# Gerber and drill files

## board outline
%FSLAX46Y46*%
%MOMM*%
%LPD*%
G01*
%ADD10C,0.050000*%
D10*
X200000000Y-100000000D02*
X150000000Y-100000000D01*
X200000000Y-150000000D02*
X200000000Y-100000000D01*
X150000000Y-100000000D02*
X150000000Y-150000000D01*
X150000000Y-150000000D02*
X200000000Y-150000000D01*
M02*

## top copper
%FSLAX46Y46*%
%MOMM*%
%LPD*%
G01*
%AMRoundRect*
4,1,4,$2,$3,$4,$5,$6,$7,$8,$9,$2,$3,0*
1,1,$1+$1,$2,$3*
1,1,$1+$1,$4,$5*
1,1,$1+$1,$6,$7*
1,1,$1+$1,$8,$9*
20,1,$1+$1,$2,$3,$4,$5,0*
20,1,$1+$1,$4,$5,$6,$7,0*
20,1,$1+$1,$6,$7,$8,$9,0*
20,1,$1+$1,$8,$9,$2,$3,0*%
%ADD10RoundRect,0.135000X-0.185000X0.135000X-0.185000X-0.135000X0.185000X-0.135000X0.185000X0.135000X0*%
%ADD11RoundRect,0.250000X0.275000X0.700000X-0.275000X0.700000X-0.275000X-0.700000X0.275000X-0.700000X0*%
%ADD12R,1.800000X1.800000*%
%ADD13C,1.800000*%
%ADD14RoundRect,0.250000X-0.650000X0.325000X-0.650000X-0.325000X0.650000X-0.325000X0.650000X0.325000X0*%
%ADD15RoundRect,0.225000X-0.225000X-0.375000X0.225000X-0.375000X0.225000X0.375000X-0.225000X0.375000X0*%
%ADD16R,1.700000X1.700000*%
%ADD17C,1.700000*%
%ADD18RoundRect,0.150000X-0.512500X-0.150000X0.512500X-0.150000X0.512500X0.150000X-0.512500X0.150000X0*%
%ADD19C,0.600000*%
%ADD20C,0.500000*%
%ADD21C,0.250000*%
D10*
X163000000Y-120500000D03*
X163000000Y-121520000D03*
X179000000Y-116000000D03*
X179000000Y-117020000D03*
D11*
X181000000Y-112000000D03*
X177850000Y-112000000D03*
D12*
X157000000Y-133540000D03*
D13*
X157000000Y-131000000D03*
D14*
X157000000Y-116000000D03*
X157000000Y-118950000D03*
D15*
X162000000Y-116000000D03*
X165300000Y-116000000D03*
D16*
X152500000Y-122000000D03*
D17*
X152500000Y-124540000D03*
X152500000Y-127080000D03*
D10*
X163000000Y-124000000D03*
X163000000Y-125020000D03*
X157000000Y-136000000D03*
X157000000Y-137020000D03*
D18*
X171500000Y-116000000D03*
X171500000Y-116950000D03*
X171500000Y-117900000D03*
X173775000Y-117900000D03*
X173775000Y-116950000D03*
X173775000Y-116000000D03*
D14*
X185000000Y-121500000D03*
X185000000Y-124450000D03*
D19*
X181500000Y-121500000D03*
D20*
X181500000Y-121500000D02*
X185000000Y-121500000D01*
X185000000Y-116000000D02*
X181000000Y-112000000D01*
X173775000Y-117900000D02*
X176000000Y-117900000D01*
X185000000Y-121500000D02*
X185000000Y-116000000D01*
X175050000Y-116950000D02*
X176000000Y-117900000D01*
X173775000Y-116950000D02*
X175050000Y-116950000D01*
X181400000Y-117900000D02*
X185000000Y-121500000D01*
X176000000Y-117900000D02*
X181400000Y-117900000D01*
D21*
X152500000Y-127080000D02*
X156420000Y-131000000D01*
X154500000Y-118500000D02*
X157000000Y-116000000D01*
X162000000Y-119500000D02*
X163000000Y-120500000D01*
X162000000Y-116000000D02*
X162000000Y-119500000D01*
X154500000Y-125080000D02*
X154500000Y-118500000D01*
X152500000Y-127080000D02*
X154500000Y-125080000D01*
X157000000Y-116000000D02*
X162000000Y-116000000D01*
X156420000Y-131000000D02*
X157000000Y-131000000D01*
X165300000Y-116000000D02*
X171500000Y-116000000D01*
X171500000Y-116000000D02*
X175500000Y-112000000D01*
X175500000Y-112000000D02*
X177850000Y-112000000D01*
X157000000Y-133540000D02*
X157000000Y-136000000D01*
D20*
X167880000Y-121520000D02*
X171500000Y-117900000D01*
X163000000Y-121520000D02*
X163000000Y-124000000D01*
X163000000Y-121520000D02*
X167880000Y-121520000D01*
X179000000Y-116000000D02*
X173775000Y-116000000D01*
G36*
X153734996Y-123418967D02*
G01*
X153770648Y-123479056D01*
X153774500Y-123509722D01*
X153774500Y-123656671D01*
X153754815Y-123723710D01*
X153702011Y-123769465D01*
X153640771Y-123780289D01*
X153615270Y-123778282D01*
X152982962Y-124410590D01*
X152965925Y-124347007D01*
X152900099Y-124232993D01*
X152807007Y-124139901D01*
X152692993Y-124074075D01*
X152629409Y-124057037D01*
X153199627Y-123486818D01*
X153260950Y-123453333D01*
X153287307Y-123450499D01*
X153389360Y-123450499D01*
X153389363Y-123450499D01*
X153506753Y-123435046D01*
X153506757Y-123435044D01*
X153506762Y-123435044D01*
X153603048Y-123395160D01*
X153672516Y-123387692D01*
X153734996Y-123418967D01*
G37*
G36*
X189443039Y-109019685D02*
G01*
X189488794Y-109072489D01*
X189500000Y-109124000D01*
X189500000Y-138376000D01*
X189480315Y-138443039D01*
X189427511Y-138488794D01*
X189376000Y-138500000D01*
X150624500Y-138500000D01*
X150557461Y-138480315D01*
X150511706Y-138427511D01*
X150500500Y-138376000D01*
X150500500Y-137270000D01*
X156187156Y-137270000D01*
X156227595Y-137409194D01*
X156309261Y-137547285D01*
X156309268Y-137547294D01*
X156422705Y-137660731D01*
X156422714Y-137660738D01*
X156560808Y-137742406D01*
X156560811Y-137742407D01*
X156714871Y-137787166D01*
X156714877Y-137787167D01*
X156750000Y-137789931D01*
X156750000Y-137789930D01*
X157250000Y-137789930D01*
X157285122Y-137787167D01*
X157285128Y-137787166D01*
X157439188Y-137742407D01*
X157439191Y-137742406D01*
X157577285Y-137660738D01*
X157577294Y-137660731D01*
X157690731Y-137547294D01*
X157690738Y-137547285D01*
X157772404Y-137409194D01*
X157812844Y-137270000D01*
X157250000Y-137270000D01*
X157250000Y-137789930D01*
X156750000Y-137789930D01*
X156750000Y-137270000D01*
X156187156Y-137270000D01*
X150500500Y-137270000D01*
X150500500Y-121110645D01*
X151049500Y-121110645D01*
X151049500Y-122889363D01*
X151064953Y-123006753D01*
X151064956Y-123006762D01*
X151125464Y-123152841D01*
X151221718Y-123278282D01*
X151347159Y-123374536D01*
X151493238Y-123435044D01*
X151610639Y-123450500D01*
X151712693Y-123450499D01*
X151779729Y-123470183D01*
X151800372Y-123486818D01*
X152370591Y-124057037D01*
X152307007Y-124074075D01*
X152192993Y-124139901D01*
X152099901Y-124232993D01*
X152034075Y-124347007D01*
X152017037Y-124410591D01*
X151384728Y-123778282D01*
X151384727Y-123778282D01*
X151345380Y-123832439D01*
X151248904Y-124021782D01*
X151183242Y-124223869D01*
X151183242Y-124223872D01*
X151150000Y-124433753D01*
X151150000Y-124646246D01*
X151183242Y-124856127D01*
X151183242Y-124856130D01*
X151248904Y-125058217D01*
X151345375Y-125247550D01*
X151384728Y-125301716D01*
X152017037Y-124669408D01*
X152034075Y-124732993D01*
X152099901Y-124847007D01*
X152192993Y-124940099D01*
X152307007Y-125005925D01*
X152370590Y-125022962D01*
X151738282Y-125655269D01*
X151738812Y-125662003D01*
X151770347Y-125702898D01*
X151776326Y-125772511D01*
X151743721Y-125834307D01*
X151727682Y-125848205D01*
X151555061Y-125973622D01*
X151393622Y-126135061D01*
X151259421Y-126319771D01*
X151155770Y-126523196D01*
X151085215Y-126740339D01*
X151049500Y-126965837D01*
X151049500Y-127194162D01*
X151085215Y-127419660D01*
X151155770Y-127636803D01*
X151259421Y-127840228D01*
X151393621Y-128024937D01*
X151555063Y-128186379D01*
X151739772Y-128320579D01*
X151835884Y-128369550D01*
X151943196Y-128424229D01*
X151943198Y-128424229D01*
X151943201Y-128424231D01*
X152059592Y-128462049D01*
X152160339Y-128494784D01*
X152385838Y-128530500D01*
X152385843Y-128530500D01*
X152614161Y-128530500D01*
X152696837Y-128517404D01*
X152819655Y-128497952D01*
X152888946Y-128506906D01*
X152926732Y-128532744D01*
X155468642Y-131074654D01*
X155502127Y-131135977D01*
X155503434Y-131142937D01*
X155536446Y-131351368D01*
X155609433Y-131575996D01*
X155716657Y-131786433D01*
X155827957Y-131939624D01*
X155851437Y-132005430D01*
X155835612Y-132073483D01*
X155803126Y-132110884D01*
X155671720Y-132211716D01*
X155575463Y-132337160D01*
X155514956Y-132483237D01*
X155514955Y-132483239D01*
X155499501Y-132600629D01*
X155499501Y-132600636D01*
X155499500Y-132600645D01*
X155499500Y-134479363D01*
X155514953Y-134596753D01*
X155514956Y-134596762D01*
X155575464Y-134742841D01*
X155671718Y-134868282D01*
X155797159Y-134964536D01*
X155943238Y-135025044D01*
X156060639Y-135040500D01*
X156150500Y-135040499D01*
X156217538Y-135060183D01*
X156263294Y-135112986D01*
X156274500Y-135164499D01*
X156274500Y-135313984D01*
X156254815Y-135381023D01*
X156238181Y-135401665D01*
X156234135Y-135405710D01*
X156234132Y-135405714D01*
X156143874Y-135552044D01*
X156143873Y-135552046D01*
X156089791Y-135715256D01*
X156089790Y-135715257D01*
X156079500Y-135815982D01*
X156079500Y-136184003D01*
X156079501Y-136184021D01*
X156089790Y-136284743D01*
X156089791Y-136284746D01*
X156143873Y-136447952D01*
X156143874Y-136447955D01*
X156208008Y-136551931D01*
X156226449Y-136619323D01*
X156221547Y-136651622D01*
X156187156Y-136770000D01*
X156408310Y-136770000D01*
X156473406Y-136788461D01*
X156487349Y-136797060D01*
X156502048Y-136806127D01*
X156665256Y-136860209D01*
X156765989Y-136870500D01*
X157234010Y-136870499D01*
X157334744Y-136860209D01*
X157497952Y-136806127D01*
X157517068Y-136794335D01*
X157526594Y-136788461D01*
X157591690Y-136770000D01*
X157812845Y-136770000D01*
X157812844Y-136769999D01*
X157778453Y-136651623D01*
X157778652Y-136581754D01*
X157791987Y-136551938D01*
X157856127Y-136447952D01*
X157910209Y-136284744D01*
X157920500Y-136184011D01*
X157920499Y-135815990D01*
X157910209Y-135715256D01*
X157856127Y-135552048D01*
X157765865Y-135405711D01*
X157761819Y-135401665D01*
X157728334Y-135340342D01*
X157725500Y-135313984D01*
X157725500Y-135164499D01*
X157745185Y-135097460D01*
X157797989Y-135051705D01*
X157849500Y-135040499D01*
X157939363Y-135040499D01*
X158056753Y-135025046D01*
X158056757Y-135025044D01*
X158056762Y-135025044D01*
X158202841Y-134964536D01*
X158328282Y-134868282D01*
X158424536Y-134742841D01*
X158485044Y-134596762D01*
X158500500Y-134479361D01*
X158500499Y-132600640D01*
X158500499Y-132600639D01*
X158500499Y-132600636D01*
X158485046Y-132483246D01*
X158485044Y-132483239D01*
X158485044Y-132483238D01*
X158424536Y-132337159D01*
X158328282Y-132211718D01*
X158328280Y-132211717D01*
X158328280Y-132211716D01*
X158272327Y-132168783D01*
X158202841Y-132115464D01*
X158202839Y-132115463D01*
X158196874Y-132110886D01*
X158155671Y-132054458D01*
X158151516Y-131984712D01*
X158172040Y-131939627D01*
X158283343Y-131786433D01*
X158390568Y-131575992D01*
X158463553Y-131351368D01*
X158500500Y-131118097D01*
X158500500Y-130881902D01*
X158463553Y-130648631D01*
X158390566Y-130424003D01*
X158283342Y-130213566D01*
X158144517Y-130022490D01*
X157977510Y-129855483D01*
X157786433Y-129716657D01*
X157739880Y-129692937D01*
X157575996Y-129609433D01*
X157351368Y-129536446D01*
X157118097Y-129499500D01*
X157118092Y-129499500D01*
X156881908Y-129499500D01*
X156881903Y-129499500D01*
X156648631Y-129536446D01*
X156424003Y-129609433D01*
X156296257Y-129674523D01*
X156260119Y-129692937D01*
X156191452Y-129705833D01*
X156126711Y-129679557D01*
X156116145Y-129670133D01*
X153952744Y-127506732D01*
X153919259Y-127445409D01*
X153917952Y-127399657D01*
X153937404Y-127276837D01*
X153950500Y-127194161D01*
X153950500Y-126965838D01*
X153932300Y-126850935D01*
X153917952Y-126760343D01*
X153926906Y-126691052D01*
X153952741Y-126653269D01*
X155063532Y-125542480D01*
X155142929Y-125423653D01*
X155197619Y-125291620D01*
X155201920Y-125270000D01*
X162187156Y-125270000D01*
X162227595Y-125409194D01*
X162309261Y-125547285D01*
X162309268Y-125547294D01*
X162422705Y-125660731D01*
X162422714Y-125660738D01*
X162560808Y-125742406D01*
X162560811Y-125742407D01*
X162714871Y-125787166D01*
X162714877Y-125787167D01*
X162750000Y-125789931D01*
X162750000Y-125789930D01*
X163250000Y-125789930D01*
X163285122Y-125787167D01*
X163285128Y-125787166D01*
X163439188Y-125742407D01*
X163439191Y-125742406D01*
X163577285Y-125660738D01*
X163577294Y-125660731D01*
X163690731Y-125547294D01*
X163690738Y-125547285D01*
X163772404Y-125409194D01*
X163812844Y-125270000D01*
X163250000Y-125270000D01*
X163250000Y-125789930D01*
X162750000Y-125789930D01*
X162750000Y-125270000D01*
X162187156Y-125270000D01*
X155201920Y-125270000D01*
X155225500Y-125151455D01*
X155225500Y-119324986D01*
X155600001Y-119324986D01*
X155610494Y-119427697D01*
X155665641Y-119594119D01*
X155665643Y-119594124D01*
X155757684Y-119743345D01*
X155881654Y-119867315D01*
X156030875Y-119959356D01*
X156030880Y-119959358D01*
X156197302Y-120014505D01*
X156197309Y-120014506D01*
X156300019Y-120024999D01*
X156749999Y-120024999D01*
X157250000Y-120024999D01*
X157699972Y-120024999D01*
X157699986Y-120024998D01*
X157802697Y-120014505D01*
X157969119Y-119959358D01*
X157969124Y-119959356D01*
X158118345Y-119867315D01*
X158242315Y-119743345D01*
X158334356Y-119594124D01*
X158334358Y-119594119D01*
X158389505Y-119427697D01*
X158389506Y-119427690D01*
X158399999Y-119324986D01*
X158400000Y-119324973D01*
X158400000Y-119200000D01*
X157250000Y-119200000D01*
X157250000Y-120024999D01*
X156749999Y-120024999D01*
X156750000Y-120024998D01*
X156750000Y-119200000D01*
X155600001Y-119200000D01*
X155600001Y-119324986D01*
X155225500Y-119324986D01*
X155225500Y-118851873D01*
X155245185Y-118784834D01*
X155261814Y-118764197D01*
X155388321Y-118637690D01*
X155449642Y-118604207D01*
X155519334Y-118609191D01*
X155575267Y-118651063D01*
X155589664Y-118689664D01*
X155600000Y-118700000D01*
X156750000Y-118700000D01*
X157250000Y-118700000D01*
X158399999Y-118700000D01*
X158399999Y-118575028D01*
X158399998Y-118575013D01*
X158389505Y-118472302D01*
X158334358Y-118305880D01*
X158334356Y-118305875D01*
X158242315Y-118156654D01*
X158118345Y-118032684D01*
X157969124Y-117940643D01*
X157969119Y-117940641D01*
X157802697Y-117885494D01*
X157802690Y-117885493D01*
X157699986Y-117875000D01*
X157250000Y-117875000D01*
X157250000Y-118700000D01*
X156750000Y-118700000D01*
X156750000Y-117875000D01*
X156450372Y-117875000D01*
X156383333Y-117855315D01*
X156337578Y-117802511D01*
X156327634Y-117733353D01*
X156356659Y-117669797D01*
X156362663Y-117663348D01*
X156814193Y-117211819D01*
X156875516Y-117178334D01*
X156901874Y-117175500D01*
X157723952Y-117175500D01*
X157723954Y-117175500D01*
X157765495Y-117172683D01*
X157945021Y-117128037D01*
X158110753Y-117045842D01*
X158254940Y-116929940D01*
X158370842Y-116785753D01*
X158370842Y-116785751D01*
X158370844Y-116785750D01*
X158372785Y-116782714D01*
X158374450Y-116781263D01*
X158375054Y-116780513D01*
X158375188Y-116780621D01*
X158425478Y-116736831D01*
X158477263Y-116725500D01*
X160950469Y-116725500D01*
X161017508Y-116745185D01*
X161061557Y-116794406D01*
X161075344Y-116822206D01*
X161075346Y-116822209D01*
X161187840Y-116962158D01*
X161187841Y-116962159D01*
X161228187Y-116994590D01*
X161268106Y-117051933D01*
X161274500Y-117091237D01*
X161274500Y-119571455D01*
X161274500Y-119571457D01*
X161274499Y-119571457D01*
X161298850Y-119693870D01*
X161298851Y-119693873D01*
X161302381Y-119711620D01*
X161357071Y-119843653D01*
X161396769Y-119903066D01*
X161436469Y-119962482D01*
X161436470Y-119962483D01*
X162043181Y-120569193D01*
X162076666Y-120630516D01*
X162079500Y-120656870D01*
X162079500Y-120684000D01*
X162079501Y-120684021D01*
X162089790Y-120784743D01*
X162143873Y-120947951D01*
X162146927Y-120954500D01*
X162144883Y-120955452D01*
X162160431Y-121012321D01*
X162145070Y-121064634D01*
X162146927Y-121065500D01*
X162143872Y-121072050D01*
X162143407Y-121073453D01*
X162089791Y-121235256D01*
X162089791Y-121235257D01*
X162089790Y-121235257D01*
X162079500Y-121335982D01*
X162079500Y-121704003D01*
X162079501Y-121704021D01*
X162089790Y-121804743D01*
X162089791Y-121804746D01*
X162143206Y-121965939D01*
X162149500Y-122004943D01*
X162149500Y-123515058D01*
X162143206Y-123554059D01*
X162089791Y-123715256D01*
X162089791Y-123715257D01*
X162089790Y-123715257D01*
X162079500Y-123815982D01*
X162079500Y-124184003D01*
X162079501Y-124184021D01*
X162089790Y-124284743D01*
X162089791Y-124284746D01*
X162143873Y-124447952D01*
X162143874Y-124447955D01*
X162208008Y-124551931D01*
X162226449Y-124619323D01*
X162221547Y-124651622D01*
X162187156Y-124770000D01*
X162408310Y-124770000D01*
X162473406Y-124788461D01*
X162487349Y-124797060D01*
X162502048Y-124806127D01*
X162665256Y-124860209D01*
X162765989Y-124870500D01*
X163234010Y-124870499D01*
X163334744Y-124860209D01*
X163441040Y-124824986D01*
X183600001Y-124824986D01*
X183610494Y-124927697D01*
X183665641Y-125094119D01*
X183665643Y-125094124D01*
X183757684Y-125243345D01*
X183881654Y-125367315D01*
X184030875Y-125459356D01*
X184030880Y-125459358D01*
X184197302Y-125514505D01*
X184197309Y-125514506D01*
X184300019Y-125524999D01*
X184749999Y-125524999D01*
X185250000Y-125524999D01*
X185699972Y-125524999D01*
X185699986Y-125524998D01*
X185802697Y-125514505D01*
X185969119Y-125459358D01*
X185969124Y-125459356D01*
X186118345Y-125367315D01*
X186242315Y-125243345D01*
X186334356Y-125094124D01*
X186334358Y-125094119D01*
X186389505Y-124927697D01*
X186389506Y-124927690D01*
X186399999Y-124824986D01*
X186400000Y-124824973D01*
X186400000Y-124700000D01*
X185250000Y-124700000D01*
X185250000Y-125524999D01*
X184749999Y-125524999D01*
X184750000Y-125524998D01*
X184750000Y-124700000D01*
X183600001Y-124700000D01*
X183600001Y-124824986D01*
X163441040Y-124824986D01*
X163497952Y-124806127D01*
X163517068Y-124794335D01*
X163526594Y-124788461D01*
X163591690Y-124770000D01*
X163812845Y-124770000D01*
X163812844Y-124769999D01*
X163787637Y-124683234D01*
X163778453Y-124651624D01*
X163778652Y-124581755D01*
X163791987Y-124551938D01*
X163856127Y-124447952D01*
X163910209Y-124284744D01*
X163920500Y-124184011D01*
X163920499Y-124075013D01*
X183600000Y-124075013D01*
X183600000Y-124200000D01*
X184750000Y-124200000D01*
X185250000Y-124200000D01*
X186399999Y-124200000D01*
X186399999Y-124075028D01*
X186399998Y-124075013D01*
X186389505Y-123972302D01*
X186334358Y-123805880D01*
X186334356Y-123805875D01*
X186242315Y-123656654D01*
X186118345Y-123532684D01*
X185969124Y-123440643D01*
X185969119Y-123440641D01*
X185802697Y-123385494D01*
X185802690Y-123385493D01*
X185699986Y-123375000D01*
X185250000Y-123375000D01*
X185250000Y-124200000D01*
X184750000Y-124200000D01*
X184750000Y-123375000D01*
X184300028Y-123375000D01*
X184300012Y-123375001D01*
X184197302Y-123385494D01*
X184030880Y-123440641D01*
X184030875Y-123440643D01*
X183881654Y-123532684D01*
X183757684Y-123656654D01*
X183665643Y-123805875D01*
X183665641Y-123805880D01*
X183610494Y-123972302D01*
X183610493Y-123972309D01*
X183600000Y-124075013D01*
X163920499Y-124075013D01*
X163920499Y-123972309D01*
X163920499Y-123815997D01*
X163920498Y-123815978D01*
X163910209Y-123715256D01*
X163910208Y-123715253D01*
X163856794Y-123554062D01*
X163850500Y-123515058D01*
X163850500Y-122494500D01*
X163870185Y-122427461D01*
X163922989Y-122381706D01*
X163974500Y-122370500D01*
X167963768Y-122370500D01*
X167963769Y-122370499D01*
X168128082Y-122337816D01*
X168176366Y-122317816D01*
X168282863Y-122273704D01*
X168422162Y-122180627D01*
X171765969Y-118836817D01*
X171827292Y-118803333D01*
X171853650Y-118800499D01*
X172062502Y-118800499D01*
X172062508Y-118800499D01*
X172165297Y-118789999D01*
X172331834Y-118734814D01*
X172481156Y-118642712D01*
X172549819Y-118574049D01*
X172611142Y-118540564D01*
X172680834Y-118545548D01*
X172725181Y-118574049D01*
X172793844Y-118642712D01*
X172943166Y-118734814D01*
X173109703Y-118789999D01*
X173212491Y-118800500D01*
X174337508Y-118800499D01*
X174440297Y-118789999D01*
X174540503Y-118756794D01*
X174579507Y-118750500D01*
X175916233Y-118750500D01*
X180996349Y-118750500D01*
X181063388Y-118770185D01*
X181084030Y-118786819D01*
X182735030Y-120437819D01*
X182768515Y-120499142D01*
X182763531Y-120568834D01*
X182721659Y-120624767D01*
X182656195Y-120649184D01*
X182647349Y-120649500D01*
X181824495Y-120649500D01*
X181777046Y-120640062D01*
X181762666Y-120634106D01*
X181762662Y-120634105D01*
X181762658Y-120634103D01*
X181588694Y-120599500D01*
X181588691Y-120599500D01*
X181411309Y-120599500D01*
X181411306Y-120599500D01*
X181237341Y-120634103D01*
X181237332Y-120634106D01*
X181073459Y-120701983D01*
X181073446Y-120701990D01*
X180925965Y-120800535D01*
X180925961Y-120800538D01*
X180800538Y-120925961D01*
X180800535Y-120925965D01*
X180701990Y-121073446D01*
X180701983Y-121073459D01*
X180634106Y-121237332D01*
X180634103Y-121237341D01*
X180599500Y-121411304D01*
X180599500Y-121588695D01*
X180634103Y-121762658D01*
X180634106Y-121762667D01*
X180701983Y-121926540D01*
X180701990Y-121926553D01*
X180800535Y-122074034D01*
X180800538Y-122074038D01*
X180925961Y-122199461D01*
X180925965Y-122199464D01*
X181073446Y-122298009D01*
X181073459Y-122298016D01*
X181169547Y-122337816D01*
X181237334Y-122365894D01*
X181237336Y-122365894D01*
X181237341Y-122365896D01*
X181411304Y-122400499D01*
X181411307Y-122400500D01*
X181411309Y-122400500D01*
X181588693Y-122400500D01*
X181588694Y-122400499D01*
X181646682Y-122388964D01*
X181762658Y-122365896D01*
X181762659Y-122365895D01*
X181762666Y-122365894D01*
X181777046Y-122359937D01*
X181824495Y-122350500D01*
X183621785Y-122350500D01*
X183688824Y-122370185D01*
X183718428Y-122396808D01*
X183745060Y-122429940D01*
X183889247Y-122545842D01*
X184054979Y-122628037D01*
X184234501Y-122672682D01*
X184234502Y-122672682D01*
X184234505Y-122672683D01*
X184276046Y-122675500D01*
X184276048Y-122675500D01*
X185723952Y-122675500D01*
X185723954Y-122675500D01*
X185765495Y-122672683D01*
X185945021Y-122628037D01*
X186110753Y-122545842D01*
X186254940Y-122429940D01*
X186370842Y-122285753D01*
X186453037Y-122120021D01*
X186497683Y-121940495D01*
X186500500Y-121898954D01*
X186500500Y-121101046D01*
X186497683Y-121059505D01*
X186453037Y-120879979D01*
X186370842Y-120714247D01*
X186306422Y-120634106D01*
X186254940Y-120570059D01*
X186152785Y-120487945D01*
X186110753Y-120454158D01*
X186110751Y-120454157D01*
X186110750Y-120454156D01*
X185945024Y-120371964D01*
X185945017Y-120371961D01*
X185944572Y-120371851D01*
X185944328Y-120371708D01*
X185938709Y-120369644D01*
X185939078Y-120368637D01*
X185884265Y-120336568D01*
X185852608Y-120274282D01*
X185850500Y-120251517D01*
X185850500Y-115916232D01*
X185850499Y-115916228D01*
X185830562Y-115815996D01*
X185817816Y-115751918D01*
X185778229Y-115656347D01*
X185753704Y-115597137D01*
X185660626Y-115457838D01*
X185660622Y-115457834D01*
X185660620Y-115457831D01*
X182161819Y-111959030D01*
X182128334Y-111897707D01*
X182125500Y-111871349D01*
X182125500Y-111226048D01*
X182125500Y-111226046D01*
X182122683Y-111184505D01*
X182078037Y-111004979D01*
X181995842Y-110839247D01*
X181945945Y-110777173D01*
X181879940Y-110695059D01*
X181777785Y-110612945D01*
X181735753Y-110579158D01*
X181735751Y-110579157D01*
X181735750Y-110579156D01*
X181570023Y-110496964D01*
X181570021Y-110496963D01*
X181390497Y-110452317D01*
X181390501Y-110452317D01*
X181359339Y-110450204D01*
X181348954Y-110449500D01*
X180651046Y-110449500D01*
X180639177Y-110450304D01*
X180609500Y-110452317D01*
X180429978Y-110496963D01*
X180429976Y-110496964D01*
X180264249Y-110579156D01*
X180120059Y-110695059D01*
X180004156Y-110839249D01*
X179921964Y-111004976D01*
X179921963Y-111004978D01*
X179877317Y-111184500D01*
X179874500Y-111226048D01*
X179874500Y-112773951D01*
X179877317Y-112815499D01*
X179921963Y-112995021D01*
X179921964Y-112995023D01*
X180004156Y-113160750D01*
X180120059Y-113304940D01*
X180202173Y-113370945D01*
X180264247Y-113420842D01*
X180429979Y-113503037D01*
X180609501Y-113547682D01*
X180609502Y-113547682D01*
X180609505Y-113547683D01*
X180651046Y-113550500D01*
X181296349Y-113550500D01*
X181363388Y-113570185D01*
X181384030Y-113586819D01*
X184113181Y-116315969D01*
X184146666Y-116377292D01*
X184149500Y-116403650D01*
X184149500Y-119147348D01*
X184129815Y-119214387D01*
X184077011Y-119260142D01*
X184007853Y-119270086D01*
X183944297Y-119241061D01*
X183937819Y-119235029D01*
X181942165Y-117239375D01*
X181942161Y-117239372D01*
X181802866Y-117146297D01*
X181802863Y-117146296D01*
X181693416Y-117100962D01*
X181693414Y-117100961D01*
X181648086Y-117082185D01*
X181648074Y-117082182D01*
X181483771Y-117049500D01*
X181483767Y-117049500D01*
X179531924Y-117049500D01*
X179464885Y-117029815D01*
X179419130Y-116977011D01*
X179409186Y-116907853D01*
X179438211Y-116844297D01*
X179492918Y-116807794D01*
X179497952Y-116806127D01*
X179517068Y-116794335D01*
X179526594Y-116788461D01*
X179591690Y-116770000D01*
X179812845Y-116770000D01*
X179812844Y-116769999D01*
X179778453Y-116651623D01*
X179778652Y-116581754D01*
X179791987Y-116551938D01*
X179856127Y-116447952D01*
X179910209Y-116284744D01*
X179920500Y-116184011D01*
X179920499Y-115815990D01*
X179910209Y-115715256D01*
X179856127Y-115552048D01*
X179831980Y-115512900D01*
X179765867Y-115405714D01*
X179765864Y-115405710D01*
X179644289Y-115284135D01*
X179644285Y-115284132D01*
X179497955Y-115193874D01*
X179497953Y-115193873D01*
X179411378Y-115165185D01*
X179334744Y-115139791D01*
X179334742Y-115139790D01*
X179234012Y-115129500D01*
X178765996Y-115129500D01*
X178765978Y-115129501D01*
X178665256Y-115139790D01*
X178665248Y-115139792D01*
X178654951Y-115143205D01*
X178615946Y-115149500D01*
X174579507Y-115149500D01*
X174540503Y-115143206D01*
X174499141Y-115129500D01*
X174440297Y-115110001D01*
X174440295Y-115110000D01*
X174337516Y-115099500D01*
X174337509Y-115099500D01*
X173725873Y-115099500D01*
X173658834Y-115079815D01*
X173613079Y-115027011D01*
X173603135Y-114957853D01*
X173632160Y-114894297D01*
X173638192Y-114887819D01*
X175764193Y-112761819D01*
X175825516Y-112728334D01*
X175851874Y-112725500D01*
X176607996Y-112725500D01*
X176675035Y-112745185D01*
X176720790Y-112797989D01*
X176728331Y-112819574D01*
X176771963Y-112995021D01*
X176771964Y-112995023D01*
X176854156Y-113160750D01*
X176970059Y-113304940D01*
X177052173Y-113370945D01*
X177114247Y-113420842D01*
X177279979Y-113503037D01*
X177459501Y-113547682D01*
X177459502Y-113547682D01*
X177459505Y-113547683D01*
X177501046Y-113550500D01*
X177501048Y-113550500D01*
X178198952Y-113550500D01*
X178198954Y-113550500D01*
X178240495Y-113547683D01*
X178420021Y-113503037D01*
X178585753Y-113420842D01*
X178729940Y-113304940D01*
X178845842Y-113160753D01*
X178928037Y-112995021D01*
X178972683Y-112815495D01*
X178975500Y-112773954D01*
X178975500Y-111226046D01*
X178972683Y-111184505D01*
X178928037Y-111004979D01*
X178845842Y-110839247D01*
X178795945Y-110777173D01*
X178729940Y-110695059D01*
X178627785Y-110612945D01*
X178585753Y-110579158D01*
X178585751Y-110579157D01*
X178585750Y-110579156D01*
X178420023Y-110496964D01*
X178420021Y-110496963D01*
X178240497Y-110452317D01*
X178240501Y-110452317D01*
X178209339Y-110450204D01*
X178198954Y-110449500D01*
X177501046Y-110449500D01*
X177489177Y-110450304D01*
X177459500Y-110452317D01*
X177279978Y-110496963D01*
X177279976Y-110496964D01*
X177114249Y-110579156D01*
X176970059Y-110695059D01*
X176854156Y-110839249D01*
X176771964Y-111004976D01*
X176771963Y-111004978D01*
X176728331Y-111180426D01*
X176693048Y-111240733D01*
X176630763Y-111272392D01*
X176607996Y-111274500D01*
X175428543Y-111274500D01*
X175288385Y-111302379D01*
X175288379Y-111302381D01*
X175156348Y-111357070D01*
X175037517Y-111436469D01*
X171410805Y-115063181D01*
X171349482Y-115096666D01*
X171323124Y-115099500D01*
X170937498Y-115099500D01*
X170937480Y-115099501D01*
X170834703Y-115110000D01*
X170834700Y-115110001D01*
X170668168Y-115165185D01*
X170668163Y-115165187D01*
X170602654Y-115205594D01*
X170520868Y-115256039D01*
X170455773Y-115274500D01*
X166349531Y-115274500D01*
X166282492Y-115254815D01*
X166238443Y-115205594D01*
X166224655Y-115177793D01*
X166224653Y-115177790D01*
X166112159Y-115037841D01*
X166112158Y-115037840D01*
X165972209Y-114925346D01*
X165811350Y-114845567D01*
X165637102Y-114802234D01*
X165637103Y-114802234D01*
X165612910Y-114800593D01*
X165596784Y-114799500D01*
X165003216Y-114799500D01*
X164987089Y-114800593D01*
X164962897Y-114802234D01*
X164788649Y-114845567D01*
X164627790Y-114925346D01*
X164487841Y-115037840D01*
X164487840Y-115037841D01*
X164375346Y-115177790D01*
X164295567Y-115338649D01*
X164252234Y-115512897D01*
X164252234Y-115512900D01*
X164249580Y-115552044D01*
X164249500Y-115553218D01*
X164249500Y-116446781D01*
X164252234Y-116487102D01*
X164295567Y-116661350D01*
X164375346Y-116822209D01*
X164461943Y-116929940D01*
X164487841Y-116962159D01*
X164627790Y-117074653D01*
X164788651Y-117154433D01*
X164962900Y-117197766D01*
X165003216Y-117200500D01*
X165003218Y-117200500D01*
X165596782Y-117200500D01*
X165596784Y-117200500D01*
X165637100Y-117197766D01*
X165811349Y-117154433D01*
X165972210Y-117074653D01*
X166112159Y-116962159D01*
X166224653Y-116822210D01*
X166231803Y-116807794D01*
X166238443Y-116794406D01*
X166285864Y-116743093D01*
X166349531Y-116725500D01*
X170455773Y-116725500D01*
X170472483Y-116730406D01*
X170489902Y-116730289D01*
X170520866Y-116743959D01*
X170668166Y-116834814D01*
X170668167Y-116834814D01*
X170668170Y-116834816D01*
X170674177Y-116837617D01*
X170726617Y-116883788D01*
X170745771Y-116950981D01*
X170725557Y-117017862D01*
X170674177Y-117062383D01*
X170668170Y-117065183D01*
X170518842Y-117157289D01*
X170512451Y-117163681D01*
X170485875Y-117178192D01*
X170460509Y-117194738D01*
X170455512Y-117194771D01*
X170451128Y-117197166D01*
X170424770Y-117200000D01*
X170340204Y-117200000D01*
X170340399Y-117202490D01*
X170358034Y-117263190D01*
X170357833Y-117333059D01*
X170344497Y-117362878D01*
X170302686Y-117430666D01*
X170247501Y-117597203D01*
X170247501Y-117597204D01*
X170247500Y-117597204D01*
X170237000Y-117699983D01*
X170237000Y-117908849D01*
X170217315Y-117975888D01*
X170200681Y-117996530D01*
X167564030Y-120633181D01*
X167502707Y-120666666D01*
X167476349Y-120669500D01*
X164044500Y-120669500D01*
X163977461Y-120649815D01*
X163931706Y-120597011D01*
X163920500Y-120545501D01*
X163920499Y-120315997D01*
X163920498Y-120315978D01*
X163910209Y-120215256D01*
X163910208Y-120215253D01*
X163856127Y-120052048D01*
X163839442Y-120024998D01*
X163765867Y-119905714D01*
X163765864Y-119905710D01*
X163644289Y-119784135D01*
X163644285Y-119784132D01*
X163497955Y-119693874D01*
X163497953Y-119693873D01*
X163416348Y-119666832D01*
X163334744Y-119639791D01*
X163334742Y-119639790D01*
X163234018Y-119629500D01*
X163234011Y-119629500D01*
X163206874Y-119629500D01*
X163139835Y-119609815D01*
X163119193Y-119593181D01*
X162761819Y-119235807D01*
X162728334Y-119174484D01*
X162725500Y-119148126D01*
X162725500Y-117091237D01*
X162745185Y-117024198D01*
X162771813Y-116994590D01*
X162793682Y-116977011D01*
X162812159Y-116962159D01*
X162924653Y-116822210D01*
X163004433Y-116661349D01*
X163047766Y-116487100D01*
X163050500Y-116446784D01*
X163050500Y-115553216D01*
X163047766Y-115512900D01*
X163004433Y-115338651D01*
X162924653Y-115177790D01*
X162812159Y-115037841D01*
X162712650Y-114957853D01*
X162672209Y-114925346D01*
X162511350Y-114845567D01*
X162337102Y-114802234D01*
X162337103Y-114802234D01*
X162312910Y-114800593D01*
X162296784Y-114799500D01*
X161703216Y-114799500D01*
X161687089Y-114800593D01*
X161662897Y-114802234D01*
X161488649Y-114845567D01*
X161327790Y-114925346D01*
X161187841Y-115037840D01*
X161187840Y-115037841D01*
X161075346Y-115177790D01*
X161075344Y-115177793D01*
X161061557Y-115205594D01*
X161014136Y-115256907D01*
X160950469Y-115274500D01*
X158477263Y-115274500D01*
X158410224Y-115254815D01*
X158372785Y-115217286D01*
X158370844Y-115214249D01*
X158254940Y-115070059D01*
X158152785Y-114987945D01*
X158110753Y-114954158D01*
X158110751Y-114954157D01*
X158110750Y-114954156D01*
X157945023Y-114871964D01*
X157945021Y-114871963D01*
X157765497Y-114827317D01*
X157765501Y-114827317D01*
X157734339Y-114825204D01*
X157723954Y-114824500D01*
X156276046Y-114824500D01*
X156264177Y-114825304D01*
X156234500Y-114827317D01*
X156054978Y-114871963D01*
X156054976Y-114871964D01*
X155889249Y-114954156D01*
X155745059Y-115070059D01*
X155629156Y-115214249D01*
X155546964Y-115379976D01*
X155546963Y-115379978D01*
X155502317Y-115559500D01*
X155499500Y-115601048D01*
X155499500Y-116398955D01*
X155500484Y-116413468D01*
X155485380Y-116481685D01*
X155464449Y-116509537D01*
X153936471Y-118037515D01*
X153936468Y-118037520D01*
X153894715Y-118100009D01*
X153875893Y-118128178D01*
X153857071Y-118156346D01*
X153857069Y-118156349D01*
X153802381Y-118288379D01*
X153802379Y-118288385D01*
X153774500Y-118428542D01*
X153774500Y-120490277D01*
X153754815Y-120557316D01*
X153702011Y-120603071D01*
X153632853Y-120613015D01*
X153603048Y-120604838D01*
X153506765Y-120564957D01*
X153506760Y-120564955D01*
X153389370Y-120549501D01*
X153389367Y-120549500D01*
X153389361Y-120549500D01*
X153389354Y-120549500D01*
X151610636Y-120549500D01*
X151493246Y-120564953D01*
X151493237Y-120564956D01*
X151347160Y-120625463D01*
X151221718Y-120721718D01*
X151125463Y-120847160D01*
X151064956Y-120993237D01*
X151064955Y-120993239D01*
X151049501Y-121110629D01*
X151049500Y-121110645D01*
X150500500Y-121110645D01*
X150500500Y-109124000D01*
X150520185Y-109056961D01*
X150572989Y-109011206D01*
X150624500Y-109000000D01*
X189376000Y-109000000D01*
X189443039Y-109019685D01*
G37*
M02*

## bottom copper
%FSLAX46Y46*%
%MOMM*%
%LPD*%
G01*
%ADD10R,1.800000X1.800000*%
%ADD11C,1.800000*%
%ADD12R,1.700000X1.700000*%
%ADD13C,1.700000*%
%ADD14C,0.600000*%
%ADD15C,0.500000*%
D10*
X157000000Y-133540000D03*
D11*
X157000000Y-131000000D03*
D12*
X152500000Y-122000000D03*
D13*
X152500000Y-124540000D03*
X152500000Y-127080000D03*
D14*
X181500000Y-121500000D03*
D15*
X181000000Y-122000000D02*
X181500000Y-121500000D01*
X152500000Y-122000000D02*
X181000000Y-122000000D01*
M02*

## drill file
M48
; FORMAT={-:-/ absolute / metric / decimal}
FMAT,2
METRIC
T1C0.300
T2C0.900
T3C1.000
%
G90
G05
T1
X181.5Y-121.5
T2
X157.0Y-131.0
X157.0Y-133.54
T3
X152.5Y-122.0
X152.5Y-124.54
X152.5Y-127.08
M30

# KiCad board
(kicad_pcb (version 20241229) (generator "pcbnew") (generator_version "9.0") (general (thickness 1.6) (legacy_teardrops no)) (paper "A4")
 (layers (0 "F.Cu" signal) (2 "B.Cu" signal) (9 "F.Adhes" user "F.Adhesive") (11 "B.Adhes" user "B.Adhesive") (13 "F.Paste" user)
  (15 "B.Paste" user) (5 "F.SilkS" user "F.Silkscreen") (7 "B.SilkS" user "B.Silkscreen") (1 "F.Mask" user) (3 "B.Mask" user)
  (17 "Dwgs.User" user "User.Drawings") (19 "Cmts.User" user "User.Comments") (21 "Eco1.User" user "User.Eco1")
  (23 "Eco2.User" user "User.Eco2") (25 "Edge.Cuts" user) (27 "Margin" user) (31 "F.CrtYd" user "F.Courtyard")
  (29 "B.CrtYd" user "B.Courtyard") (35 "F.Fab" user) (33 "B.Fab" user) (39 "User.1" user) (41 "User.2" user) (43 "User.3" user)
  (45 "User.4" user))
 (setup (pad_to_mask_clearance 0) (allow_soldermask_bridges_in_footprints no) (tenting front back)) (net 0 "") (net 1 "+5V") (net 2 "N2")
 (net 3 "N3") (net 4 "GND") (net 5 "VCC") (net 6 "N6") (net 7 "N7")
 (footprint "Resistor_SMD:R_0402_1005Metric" (layer "F.Cu") (at 163 121.01 -90)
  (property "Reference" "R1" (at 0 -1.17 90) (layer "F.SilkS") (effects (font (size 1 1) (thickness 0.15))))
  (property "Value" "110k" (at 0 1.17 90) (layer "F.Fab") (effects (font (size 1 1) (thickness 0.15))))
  (pad "1" smd roundrect (at -0.51 0 270) (size 0.54 0.64) (layers "F.Cu" "F.Mask" "F.Paste") (roundrect_rratio 0.25) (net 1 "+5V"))
  (pad "2" smd roundrect (at 0.51 0 270) (size 0.54 0.64) (layers "F.Cu" "F.Mask" "F.Paste") (roundrect_rratio 0.25) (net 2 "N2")))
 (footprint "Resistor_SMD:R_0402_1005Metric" (layer "F.Cu") (at 179 116.51 -90)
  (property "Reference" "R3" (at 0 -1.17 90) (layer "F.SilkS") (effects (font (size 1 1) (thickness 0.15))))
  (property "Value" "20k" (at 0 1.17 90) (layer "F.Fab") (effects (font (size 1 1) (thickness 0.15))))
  (pad "1" smd roundrect (at -0.51 0 270) (size 0.54 0.64) (layers "F.Cu" "F.Mask" "F.Paste") (roundrect_rratio 0.25) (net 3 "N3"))
  (pad "2" smd roundrect (at 0.51 0 270) (size 0.54 0.64) (layers "F.Cu" "F.Mask" "F.Paste") (roundrect_rratio 0.25) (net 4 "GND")))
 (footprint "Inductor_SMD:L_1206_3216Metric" (layer "F.Cu") (at 179.425 112 180)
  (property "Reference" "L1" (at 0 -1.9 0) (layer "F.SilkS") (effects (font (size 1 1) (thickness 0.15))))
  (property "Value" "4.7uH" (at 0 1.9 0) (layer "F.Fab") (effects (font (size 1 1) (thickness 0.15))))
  (pad "1" smd roundrect (at -1.575 0 180) (size 1.05 1.9) (layers "F.Cu" "F.Mask" "F.Paste") (roundrect_rratio 0.238095) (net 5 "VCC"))
  (pad "2" smd roundrect (at 1.575 0 180) (size 1.05 1.9) (layers "F.Cu" "F.Mask" "F.Paste") (roundrect_rratio 0.238095) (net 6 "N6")))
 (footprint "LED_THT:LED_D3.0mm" (layer "F.Cu") (at 157 133.54 90)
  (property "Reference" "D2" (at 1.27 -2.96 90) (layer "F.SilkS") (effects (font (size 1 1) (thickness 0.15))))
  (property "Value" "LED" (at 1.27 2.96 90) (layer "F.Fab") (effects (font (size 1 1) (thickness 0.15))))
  (pad "1" thru_hole rect (at 0 0 90) (size 1.8 1.8) (drill 0.9) (layers "*.Cu" "*.Mask") (remove_unused_layers no) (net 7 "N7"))
  (pad "2" thru_hole circle (at 2.54 0 90) (size 1.8 1.8) (drill 0.9) (layers "*.Cu" "*.Mask") (remove_unused_layers no) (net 1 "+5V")))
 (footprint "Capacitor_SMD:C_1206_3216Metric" (layer "F.Cu") (at 157 117.475 -90)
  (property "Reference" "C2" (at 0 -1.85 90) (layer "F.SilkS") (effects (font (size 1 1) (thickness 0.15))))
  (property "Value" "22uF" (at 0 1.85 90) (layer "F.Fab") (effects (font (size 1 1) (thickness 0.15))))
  (pad "1" smd roundrect (at -1.475 0 270) (size 1.15 1.8) (layers "F.Cu" "F.Mask" "F.Paste") (roundrect_rratio 0.217391) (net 1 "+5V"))
  (pad "2" smd roundrect (at 1.475 0 270) (size 1.15 1.8) (layers "F.Cu" "F.Mask" "F.Paste") (roundrect_rratio 0.217391) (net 4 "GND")))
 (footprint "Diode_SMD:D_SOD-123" (layer "F.Cu") (at 163.65 116)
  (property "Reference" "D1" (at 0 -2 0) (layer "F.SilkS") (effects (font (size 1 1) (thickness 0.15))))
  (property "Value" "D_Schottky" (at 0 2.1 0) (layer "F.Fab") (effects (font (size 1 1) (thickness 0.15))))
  (pad "1" smd roundrect (at -1.65 0) (size 0.9 1.2) (layers "F.Cu" "F.Mask" "F.Paste") (roundrect_rratio 0.25) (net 1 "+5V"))
  (pad "2" smd roundrect (at 1.65 0) (size 0.9 1.2) (layers "F.Cu" "F.Mask" "F.Paste") (roundrect_rratio 0.25) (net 6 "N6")))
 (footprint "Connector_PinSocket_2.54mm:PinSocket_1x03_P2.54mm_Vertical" (layer "F.Cu") (at 152.5 122)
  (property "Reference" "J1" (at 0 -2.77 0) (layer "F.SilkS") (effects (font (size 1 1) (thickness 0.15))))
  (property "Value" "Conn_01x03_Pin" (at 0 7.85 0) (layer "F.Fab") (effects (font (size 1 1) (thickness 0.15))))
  (pad "1" thru_hole rect (at 0 0) (size 1.7 1.7) (drill 1) (layers "*.Cu" "*.Mask") (remove_unused_layers no) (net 5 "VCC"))
  (pad "2" thru_hole circle (at 0 2.54) (size 1.7 1.7) (drill 1) (layers "*.Cu" "*.Mask") (remove_unused_layers no) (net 4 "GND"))
  (pad "3" thru_hole circle (at 0 5.08) (size 1.7 1.7) (drill 1) (layers "*.Cu" "*.Mask") (remove_unused_layers no) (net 1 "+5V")))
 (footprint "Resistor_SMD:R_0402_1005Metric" (layer "F.Cu") (at 163 124.51 -90)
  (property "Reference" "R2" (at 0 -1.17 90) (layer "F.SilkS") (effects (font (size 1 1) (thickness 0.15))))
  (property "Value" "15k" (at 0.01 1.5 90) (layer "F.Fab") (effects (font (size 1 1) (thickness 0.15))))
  (pad "1" smd roundrect (at -0.51 0 270) (size 0.54 0.64) (layers "F.Cu" "F.Mask" "F.Paste") (roundrect_rratio 0.25) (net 2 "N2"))
  (pad "2" smd roundrect (at 0.51 0 270) (size 0.54 0.64) (layers "F.Cu" "F.Mask" "F.Paste") (roundrect_rratio 0.25) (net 4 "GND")))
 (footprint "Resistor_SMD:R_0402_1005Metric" (layer "F.Cu") (at 157 136.51 -90)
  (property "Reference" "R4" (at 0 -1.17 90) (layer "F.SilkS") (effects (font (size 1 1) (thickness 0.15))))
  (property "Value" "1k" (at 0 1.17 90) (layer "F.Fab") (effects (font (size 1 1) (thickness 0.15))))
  (pad "1" smd roundrect (at -0.51 0 270) (size 0.54 0.64) (layers "F.Cu" "F.Mask" "F.Paste") (roundrect_rratio 0.25) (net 7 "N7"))
  (pad "2" smd roundrect (at 0.51 0 270) (size 0.54 0.64) (layers "F.Cu" "F.Mask" "F.Paste") (roundrect_rratio 0.25) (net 4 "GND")))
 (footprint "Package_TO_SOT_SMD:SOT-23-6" (layer "F.Cu") (at 172.6375 116.95)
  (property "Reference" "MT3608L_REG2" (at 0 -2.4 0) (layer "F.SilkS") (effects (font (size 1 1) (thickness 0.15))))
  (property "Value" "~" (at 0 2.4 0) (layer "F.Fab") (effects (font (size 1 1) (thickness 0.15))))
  (pad "1" smd roundrect (at -1.1375 -0.95) (size 1.325 0.6) (layers "F.Cu" "F.Mask" "F.Paste") (roundrect_rratio 0.25) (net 6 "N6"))
  (pad "2" smd roundrect (at -1.1375 0) (size 1.325 0.6) (layers "F.Cu" "F.Mask" "F.Paste") (roundrect_rratio 0.25) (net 4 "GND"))
  (pad "3" smd roundrect (at -1.1375 0.95) (size 1.325 0.6) (layers "F.Cu" "F.Mask" "F.Paste") (roundrect_rratio 0.25) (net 2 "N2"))
  (pad "4" smd roundrect (at 1.1375 0.95) (size 1.325 0.6) (layers "F.Cu" "F.Mask" "F.Paste") (roundrect_rratio 0.25) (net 5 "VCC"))
  (pad "5" smd roundrect (at 1.1375 0) (size 1.325 0.6) (layers "F.Cu" "F.Mask" "F.Paste") (roundrect_rratio 0.25) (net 5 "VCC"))
  (pad "6" smd roundrect (at 1.1375 -0.95) (size 1.325 0.6) (layers "F.Cu" "F.Mask" "F.Paste") (roundrect_rratio 0.25) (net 3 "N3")))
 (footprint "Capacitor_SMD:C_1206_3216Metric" (layer "F.Cu") (at 185 122.975 -90)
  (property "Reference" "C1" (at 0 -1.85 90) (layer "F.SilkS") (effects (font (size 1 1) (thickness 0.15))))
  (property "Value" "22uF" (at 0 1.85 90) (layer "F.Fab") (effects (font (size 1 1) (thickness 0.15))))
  (pad "1" smd roundrect (at -1.475 0 270) (size 1.15 1.8) (layers "F.Cu" "F.Mask" "F.Paste") (roundrect_rratio 0.217391) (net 5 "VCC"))
  (pad "2" smd roundrect (at 1.475 0 270) (size 1.15 1.8) (layers "F.Cu" "F.Mask" "F.Paste") (roundrect_rratio 0.217391) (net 4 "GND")))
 (gr_line (start 200 100) (end 150 100) (stroke (width 0.05) (type default)) (layer "Edge.Cuts"))
 (gr_line (start 200 150) (end 200 100) (stroke (width 0.05) (type default)) (layer "Edge.Cuts"))
 (gr_line (start 150 100) (end 150 150) (stroke (width 0.05) (type default)) (layer "Edge.Cuts"))
 (gr_line (start 150 150) (end 200 150) (stroke (width 0.05) (type default)) (layer "Edge.Cuts"))
 (segment (start 181.5 121.5) (end 185 121.5) (width 0.5) (layer "F.Cu") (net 5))
 (segment (start 185 116) (end 181 112) (width 0.5) (layer "F.Cu") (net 5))
 (segment (start 173.775 117.9) (end 176 117.9) (width 0.5) (layer "F.Cu") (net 5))
 (segment (start 185 121.5) (end 185 116) (width 0.5) (layer "F.Cu") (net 5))
 (segment (start 175.05 116.95) (end 176 117.9) (width 0.5) (layer "F.Cu") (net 5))
 (segment (start 173.775 116.95) (end 175.05 116.95) (width 0.5) (layer "F.Cu") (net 5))
 (segment (start 181.4 117.9) (end 185 121.5) (width 0.5) (layer "F.Cu") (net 5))
 (segment (start 176 117.9) (end 181.4 117.9) (width 0.5) (layer "F.Cu") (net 5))
 (via (at 181.5 121.5) (size 0.6) (drill 0.3) (layers "F.Cu" "B.Cu") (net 5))
 (segment (start 181 122) (end 181.5 121.5) (width 0.5) (layer "B.Cu") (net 5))
 (segment (start 152.5 122) (end 181 122) (width 0.5) (layer "B.Cu") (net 5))
 (segment (start 152.5 127.08) (end 156.42 131) (width 0.25) (layer "F.Cu") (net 1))
 (segment (start 154.5 118.5) (end 157 116) (width 0.25) (layer "F.Cu") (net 1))
 (segment (start 162 119.5) (end 163 120.5) (width 0.25) (layer "F.Cu") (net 1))
 (segment (start 162 116) (end 162 119.5) (width 0.25) (layer "F.Cu") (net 1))
 (segment (start 154.5 125.08) (end 154.5 118.5) (width 0.25) (layer "F.Cu") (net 1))
 (segment (start 152.5 127.08) (end 154.5 125.08) (width 0.25) (layer "F.Cu") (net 1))
 (segment (start 157 116) (end 162 116) (width 0.25) (layer "F.Cu") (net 1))
 (segment (start 156.42 131) (end 157 131) (width 0.25) (layer "F.Cu") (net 1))
 (segment (start 165.3 116) (end 171.5 116) (width 0.25) (layer "F.Cu") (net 6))
 (segment (start 171.5 116) (end 175.5 112) (width 0.25) (layer "F.Cu") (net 6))
 (segment (start 175.5 112) (end 177.85 112) (width 0.25) (layer "F.Cu") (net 6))
 (segment (start 157 133.54) (end 157 136) (width 0.25) (layer "F.Cu") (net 7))
 (segment (start 167.88 121.52) (end 171.5 117.9) (width 0.5) (layer "F.Cu") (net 2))
 (segment (start 163 121.52) (end 163 124) (width 0.5) (layer "F.Cu") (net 2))
 (segment (start 163 121.52) (end 167.88 121.52) (width 0.5) (layer "F.Cu") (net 2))
 (segment (start 179 116) (end 173.775 116) (width 0.5) (layer "F.Cu") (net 3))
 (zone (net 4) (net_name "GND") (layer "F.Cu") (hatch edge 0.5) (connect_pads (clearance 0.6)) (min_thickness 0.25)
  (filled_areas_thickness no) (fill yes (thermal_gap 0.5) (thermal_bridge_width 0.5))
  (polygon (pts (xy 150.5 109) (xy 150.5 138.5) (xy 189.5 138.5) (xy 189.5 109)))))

